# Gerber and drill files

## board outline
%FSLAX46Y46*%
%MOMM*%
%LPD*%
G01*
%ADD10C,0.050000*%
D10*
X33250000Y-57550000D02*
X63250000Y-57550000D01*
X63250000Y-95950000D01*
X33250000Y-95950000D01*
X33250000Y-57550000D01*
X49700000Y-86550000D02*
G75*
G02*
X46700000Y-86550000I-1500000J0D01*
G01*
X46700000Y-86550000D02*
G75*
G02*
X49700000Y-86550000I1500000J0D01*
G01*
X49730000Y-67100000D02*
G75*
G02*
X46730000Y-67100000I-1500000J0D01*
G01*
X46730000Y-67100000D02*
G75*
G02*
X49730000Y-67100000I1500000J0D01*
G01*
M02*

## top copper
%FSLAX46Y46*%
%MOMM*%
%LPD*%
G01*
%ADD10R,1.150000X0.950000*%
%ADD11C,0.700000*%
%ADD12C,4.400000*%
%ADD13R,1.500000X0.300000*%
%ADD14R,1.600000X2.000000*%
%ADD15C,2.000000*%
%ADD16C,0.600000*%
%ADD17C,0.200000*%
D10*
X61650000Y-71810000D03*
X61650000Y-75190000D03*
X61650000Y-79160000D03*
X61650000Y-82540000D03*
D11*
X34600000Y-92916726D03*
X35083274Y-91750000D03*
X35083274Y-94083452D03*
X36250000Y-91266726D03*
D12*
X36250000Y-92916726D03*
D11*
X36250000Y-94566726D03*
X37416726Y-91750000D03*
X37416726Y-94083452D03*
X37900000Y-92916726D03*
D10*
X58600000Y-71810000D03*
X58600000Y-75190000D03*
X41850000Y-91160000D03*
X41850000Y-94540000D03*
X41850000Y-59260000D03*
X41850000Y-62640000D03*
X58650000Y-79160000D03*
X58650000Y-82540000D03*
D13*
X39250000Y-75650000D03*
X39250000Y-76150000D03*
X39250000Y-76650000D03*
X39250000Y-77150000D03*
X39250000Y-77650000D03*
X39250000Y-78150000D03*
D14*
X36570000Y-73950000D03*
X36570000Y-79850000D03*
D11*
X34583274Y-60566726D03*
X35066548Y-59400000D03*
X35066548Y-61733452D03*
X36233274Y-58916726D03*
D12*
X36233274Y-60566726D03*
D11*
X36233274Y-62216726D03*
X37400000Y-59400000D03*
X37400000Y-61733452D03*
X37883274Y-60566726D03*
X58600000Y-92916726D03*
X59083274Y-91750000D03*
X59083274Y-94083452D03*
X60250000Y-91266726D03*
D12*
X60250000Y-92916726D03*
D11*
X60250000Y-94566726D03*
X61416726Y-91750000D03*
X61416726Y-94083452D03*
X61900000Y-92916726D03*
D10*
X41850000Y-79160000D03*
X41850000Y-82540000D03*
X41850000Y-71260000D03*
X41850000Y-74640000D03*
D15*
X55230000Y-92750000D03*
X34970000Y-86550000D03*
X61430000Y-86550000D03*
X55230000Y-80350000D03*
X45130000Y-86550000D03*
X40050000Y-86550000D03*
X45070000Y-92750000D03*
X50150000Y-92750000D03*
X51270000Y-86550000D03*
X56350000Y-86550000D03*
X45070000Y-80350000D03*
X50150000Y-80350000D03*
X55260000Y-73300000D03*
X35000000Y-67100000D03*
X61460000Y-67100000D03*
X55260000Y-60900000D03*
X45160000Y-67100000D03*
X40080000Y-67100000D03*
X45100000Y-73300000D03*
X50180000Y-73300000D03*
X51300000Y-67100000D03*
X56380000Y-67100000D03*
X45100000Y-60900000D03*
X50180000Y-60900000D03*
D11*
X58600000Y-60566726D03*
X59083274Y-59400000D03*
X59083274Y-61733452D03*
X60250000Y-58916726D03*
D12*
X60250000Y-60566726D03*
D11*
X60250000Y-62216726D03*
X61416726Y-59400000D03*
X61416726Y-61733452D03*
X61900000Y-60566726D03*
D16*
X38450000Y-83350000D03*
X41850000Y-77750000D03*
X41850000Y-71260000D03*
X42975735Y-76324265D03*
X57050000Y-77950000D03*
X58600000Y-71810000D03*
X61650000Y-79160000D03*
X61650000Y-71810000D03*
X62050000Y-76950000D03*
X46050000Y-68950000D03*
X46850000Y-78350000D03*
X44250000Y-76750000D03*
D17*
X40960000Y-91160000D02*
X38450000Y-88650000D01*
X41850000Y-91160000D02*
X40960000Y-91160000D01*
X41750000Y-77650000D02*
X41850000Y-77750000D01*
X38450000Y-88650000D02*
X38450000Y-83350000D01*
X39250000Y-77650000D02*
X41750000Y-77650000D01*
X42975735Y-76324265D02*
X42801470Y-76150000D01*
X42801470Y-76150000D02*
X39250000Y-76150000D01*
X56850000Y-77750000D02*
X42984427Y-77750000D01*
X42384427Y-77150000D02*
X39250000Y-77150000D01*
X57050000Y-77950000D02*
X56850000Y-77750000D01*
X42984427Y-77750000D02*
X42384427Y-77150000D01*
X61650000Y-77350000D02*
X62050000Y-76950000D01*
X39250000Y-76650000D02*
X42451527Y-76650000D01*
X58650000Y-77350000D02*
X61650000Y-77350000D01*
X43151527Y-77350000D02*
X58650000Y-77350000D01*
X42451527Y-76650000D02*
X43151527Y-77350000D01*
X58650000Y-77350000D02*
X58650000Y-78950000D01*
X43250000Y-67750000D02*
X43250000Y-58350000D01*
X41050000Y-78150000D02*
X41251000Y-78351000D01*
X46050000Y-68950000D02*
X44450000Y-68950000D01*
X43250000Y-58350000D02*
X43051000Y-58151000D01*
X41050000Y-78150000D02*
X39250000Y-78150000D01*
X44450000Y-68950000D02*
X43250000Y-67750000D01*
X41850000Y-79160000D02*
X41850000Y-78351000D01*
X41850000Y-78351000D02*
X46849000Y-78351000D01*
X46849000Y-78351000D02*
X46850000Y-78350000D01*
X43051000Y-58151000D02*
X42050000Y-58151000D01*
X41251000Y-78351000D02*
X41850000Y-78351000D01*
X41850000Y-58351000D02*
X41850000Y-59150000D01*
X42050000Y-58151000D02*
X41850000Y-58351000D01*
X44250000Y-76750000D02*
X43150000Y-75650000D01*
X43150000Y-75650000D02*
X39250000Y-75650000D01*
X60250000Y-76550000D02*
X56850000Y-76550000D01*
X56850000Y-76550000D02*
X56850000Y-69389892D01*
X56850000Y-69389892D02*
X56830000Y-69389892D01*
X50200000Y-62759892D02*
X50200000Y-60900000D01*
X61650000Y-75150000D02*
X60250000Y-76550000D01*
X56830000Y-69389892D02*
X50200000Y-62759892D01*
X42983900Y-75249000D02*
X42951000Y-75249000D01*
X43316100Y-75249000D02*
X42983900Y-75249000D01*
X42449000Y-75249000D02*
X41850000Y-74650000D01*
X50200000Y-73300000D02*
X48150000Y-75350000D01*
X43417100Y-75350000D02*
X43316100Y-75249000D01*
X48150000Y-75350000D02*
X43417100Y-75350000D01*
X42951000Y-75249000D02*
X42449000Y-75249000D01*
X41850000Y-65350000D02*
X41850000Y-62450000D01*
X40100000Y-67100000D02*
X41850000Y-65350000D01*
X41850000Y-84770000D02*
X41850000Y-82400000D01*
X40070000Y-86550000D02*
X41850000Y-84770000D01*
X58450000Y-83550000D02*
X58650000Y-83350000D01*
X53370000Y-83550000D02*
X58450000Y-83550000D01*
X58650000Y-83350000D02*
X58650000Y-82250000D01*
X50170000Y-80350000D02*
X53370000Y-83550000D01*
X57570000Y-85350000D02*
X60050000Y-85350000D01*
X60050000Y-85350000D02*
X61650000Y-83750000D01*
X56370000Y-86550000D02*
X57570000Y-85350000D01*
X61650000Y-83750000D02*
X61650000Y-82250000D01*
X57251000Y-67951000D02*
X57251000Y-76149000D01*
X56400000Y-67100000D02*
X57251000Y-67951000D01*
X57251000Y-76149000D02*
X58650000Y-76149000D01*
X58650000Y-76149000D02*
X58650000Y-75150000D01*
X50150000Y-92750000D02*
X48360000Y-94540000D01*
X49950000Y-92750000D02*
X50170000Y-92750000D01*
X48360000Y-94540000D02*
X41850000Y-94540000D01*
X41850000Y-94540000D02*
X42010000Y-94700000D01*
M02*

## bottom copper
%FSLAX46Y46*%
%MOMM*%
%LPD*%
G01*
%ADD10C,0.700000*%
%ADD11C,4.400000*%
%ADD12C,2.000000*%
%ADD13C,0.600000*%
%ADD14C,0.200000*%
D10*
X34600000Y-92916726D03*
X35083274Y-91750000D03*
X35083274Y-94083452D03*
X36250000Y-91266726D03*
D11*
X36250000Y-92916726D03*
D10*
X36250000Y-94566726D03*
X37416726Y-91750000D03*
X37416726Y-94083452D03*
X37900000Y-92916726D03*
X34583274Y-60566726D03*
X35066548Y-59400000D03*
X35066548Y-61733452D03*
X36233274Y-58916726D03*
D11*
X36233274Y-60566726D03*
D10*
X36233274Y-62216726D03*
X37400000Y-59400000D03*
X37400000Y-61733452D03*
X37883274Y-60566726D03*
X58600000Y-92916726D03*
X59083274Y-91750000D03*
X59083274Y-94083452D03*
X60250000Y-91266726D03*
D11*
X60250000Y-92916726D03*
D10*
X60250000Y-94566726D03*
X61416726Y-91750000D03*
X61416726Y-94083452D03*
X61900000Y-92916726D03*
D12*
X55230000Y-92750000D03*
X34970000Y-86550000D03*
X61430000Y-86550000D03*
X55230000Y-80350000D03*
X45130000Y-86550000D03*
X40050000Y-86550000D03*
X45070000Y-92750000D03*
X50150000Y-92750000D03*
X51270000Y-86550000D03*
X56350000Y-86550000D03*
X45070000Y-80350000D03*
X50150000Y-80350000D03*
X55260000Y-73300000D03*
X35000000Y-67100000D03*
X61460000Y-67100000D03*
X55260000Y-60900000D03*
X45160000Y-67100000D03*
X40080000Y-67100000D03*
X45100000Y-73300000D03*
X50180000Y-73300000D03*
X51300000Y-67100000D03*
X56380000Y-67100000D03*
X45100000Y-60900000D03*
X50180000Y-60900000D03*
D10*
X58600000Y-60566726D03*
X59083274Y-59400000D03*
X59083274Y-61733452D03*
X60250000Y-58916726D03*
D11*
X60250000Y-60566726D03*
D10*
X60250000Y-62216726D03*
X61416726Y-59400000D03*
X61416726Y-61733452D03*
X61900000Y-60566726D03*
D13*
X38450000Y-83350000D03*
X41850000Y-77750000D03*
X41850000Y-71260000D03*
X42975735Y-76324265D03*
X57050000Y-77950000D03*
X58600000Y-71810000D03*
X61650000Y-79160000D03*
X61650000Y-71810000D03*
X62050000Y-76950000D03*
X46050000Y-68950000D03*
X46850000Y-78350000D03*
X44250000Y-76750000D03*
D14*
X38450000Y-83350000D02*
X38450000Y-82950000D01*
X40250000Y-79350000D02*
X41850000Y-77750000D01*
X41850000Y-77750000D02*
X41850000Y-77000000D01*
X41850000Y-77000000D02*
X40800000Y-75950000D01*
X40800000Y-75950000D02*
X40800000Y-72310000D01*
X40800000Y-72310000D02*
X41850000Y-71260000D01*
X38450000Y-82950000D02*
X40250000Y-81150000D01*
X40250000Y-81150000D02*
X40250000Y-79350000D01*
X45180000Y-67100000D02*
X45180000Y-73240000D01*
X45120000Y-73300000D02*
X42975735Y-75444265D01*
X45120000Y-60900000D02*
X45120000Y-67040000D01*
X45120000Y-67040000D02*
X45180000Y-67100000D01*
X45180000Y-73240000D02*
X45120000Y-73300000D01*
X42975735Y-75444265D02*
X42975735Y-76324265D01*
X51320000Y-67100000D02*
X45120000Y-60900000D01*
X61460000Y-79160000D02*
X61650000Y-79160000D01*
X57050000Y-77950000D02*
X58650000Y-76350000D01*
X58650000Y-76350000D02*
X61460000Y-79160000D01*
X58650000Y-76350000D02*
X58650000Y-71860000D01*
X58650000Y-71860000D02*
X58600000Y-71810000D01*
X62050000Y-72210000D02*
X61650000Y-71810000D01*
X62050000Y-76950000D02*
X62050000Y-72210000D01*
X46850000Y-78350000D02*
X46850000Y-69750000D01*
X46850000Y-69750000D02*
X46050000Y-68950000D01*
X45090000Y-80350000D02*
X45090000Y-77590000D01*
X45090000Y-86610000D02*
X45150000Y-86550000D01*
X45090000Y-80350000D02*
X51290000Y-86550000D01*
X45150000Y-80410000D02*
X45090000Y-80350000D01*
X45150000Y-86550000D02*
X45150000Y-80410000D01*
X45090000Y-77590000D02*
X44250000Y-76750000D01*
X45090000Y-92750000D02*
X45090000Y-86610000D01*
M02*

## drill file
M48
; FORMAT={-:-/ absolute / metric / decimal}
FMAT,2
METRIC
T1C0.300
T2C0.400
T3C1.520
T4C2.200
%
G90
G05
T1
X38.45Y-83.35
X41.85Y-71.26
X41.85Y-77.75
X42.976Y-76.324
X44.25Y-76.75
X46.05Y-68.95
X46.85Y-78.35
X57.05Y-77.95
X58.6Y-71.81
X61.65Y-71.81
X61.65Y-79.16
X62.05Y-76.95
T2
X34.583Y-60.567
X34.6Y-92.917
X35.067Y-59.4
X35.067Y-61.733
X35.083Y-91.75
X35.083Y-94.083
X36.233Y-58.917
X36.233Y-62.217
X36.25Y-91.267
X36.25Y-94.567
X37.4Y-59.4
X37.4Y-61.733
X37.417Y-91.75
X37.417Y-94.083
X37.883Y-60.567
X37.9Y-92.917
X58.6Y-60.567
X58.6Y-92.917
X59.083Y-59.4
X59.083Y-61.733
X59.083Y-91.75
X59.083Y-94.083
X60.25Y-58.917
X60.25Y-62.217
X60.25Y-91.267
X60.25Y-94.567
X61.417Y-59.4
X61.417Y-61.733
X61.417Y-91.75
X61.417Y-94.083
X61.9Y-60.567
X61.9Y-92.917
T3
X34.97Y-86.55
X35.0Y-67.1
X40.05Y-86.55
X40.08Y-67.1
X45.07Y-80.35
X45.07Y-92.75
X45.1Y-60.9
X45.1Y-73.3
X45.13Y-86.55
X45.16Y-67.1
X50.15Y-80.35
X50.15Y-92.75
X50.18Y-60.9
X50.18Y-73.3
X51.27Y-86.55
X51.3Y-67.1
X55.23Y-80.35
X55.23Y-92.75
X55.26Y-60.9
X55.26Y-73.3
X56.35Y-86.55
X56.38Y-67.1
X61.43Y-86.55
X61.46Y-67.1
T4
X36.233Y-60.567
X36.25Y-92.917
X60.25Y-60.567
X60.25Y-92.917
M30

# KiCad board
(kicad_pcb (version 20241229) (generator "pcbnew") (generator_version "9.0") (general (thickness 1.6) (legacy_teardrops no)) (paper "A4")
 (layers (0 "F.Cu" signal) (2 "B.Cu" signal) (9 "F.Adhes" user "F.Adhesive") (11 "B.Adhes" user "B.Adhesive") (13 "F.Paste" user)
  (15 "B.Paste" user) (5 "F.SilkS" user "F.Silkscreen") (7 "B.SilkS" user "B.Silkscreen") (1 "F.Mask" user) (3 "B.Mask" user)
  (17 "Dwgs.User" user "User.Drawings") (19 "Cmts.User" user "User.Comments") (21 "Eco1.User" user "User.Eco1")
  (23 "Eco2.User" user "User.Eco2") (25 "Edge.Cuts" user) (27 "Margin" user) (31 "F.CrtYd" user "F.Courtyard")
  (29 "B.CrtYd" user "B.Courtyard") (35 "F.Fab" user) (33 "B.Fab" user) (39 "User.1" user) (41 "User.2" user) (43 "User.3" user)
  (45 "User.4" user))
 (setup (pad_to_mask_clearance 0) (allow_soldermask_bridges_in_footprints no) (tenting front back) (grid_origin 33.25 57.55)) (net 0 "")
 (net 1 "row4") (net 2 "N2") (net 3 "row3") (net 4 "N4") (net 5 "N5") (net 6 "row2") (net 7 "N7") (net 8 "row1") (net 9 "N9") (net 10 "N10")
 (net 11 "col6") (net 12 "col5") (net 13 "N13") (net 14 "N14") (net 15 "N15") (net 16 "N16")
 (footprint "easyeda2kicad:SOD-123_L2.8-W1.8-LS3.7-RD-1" (layer "F.Cu") (at 61.65 73.5 -90)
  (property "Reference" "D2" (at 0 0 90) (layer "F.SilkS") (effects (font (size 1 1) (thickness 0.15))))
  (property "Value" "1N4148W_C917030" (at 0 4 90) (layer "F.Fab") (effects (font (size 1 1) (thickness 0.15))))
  (pad "1" smd rect (at -1.69 0 270) (size 0.95 1.15) (layers "F.Cu" "F.Mask" "F.Paste") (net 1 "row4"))
  (pad "2" smd rect (at 1.69 0 270) (size 0.95 1.15) (layers "F.Cu" "F.Mask" "F.Paste") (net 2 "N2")))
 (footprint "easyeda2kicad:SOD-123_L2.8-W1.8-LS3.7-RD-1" (layer "F.Cu") (at 61.65 80.85 -90)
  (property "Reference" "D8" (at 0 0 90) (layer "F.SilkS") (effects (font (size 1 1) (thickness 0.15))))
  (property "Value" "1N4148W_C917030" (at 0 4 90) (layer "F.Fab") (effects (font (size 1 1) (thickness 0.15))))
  (pad "1" smd rect (at -1.69 0 270) (size 0.95 1.15) (layers "F.Cu" "F.Mask" "F.Paste") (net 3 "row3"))
  (pad "2" smd rect (at 1.69 0 270) (size 0.95 1.15) (layers "F.Cu" "F.Mask" "F.Paste") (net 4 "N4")))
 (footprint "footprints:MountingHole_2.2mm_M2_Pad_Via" (layer "F.Cu") (at 36.25 92.916726)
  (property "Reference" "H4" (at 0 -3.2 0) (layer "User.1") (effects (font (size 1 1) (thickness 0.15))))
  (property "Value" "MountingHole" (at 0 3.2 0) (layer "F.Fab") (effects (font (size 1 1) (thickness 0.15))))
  (pad "1" thru_hole circle (at -1.65 0) (size 0.7 0.7) (drill 0.4) (layers "*.Cu" "*.Mask") (remove_unused_layers no) (zone_connect 2))
  (pad "1" thru_hole circle (at -1.166726 -1.166726) (size 0.7 0.7) (drill 0.4) (layers "*.Cu" "*.Mask") (remove_unused_layers no)
   (zone_connect 2))
  (pad "1" thru_hole circle (at -1.166726 1.166726) (size 0.7 0.7) (drill 0.4) (layers "*.Cu" "*.Mask") (remove_unused_layers no)
   (zone_connect 2))
  (pad "1" thru_hole circle (at 0 -1.65) (size 0.7 0.7) (drill 0.4) (layers "*.Cu" "*.Mask") (remove_unused_layers no) (zone_connect 2))
  (pad "1" thru_hole circle (at 0 0) (size 4.4 4.4) (drill 2.2) (layers "*.Cu" "*.Mask") (remove_unused_layers no))
  (pad "1" thru_hole circle (at 0 1.65) (size 0.7 0.7) (drill 0.4) (layers "*.Cu" "*.Mask") (remove_unused_layers no) (zone_connect 2))
  (pad "1" thru_hole circle (at 1.166726 -1.166726) (size 0.7 0.7) (drill 0.4) (layers "*.Cu" "*.Mask") (remove_unused_layers no)
   (zone_connect 2))
  (pad "1" thru_hole circle (at 1.166726 1.166726) (size 0.7 0.7) (drill 0.4) (layers "*.Cu" "*.Mask") (remove_unused_layers no)
   (zone_connect 2))
  (pad "1" thru_hole circle (at 1.65 0) (size 0.7 0.7) (drill 0.4) (layers "*.Cu" "*.Mask") (remove_unused_layers no) (zone_connect 2)))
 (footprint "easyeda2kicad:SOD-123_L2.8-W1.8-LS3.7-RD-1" (layer "F.Cu") (at 58.6 73.5 -90)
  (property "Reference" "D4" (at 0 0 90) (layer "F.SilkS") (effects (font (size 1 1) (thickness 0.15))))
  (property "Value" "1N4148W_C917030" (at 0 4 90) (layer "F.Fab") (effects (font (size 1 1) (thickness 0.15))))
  (pad "1" smd rect (at -1.69 0 270) (size 0.95 1.15) (layers "F.Cu" "F.Mask" "F.Paste") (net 3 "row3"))
  (pad "2" smd rect (at 1.69 0 270) (size 0.95 1.15) (layers "F.Cu" "F.Mask" "F.Paste") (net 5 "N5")))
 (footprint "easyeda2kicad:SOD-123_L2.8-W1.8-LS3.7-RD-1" (layer "F.Cu") (at 41.85 92.85 -90)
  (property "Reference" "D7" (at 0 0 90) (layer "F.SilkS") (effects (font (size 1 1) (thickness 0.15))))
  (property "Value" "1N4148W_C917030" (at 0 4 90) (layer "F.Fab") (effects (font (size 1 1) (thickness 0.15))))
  (pad "1" smd rect (at -1.69 0 270) (size 0.95 1.15) (layers "F.Cu" "F.Mask" "F.Paste") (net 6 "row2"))
  (pad "2" smd rect (at 1.69 0 270) (size 0.95 1.15) (layers "F.Cu" "F.Mask" "F.Paste") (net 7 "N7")))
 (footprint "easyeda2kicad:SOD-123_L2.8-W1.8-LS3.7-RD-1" (layer "F.Cu") (at 41.85 60.95 -90)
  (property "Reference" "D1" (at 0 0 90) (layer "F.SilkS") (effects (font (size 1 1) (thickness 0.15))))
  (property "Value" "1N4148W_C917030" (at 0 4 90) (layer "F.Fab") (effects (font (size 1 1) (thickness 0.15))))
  (pad "1" smd rect (at -1.69 0 270) (size 0.95 1.15) (layers "F.Cu" "F.Mask" "F.Paste") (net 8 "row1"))
  (pad "2" smd rect (at 1.69 0 270) (size 0.95 1.15) (layers "F.Cu" "F.Mask" "F.Paste") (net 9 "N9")))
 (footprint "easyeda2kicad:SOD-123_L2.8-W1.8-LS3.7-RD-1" (layer "F.Cu") (at 58.65 80.85 -90)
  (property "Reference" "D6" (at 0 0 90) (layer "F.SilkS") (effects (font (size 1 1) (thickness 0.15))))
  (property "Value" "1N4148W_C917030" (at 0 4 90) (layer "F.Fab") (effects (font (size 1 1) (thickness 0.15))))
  (pad "1" smd rect (at -1.69 0 270) (size 0.95 1.15) (layers "F.Cu" "F.Mask" "F.Paste") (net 1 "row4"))
  (pad "2" smd rect (at 1.69 0 270) (size 0.95 1.15) (layers "F.Cu" "F.Mask" "F.Paste") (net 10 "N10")))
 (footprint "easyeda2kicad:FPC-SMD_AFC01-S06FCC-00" (layer "F.Cu") (at 37.91 76.9 -90)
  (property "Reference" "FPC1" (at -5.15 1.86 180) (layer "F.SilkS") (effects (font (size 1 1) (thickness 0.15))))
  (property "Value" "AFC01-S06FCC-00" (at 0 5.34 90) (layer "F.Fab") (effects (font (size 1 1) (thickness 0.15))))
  (pad "1" smd rect (at -1.25 -1.34 270) (size 0.3 1.5) (layers "F.Cu" "F.Mask" "F.Paste") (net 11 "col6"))
  (pad "2" smd rect (at -0.75 -1.34 270) (size 0.3 1.5) (layers "F.Cu" "F.Mask" "F.Paste") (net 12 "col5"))
  (pad "3" smd rect (at -0.25 -1.34 270) (size 0.3 1.5) (layers "F.Cu" "F.Mask" "F.Paste") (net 1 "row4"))
  (pad "4" smd rect (at 0.25 -1.34 270) (size 0.3 1.5) (layers "F.Cu" "F.Mask" "F.Paste") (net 3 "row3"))
  (pad "5" smd rect (at 0.75 -1.34 270) (size 0.3 1.5) (layers "F.Cu" "F.Mask" "F.Paste") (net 6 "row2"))
  (pad "6" smd rect (at 1.25 -1.34 270) (size 0.3 1.5) (layers "F.Cu" "F.Mask" "F.Paste") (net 8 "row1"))
  (pad "7" smd rect (at -2.95 1.34 270) (size 2 1.6) (layers "F.Cu" "F.Mask" "F.Paste") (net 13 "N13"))
  (pad "8" smd rect (at 2.95 1.34 90) (size 2 1.6) (layers "F.Cu" "F.Mask" "F.Paste") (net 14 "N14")))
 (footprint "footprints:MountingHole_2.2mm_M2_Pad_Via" (layer "F.Cu") (at 36.233274 60.566726)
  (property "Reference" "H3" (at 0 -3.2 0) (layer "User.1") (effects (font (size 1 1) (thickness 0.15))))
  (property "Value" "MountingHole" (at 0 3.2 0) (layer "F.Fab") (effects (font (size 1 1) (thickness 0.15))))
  (pad "1" thru_hole circle (at -1.65 0) (size 0.7 0.7) (drill 0.4) (layers "*.Cu" "*.Mask") (remove_unused_layers no) (zone_connect 2))
  (pad "1" thru_hole circle (at -1.166726 -1.166726) (size 0.7 0.7) (drill 0.4) (layers "*.Cu" "*.Mask") (remove_unused_layers no)
   (zone_connect 2))
  (pad "1" thru_hole circle (at -1.166726 1.166726) (size 0.7 0.7) (drill 0.4) (layers "*.Cu" "*.Mask") (remove_unused_layers no)
   (zone_connect 2))
  (pad "1" thru_hole circle (at 0 -1.65) (size 0.7 0.7) (drill 0.4) (layers "*.Cu" "*.Mask") (remove_unused_layers no) (zone_connect 2))
  (pad "1" thru_hole circle (at 0 0) (size 4.4 4.4) (drill 2.2) (layers "*.Cu" "*.Mask") (remove_unused_layers no))
  (pad "1" thru_hole circle (at 0 1.65) (size 0.7 0.7) (drill 0.4) (layers "*.Cu" "*.Mask") (remove_unused_layers no) (zone_connect 2))
  (pad "1" thru_hole circle (at 1.166726 -1.166726) (size 0.7 0.7) (drill 0.4) (layers "*.Cu" "*.Mask") (remove_unused_layers no)
   (zone_connect 2))
  (pad "1" thru_hole circle (at 1.166726 1.166726) (size 0.7 0.7) (drill 0.4) (layers "*.Cu" "*.Mask") (remove_unused_layers no)
   (zone_connect 2))
  (pad "1" thru_hole circle (at 1.65 0) (size 0.7 0.7) (drill 0.4) (layers "*.Cu" "*.Mask") (remove_unused_layers no) (zone_connect 2)))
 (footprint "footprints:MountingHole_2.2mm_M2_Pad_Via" (layer "F.Cu") (at 60.25 92.916726)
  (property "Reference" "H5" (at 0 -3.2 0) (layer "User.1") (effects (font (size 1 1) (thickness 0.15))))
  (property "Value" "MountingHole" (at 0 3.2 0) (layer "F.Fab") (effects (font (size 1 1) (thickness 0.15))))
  (pad "1" thru_hole circle (at -1.65 0) (size 0.7 0.7) (drill 0.4) (layers "*.Cu" "*.Mask") (remove_unused_layers no) (zone_connect 2))
  (pad "1" thru_hole circle (at -1.166726 -1.166726) (size 0.7 0.7) (drill 0.4) (layers "*.Cu" "*.Mask") (remove_unused_layers no)
   (zone_connect 2))
  (pad "1" thru_hole circle (at -1.166726 1.166726) (size 0.7 0.7) (drill 0.4) (layers "*.Cu" "*.Mask") (remove_unused_layers no)
   (zone_connect 2))
  (pad "1" thru_hole circle (at 0 -1.65) (size 0.7 0.7) (drill 0.4) (layers "*.Cu" "*.Mask") (remove_unused_layers no) (zone_connect 2))
  (pad "1" thru_hole circle (at 0 0) (size 4.4 4.4) (drill 2.2) (layers "*.Cu" "*.Mask") (remove_unused_layers no))
  (pad "1" thru_hole circle (at 0 1.65) (size 0.7 0.7) (drill 0.4) (layers "*.Cu" "*.Mask") (remove_unused_layers no) (zone_connect 2))
  (pad "1" thru_hole circle (at 1.166726 -1.166726) (size 0.7 0.7) (drill 0.4) (layers "*.Cu" "*.Mask") (remove_unused_layers no)
   (zone_connect 2))
  (pad "1" thru_hole circle (at 1.166726 1.166726) (size 0.7 0.7) (drill 0.4) (layers "*.Cu" "*.Mask") (remove_unused_layers no)
   (zone_connect 2))
  (pad "1" thru_hole circle (at 1.65 0) (size 0.7 0.7) (drill 0.4) (layers "*.Cu" "*.Mask") (remove_unused_layers no) (zone_connect 2)))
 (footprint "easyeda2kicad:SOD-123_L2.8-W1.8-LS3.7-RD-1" (layer "F.Cu") (at 41.85 80.85 -90)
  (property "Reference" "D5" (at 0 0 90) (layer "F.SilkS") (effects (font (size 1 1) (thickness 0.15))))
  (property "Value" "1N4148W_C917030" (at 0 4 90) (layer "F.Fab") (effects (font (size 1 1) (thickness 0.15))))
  (pad "1" smd rect (at -1.69 0 270) (size 0.95 1.15) (layers "F.Cu" "F.Mask" "F.Paste") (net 8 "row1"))
  (pad "2" smd rect (at 1.69 0 270) (size 0.95 1.15) (layers "F.Cu" "F.Mask" "F.Paste") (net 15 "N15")))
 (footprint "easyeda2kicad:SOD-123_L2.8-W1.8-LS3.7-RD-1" (layer "F.Cu") (at 41.85 72.95 -90)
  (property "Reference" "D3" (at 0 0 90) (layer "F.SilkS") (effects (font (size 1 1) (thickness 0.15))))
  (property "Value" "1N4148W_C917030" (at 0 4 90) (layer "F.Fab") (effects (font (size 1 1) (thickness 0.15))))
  (pad "1" smd rect (at -1.69 0 270) (size 0.95 1.15) (layers "F.Cu" "F.Mask" "F.Paste") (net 6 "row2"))
  (pad "2" smd rect (at 1.69 0 270) (size 0.95 1.15) (layers "F.Cu" "F.Mask" "F.Paste") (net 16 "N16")))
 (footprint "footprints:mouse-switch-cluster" (layer "F.Cu") (at 48.2 86.55 90)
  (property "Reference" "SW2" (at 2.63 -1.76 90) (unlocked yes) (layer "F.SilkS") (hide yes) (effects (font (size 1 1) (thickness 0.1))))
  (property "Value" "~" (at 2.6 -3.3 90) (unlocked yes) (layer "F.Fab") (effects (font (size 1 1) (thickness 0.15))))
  (fp_circle (center 0 0) (end 1.5 0) (stroke (width 0.05) (type default)) (fill no) (layer "Edge.Cuts"))
  (pad "" thru_hole circle (at -6.2 7.03 90) (size 2 2) (drill 1.52) (layers "*.Cu" "*.Mask") (remove_unused_layers no))
  (pad "" thru_hole circle (at 0 -13.23 270) (size 2 2) (drill 1.52) (layers "*.Cu" "*.Mask") (remove_unused_layers no))
  (pad "" thru_hole circle (at 0 13.23 90) (size 2 2) (drill 1.52) (layers "*.Cu" "*.Mask") (remove_unused_layers no))
  (pad "" thru_hole circle (at 6.2 7.03 90) (size 2 2) (drill 1.52) (layers "*.Cu" "*.Mask") (remove_unused_layers no))
  (pad "1" thru_hole circle (at 0 -3.07 270) (size 2 2) (drill 1.52) (layers "*.Cu" "*.Mask") (remove_unused_layers no) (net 11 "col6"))
  (pad "2" thru_hole circle (at 0 -8.15 270) (size 2 2) (drill 1.52) (layers "*.Cu" "*.Mask") (remove_unused_layers no) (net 15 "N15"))
  (pad "3" thru_hole circle (at -6.2 -3.13 90) (size 2 2) (drill 1.52) (layers "*.Cu" "*.Mask") (remove_unused_layers no) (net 11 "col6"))
  (pad "4" thru_hole circle (at -6.2 1.95 90) (size 2 2) (drill 1.52) (layers "*.Cu" "*.Mask") (remove_unused_layers no) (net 7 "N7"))
  (pad "5" thru_hole circle (at 0 3.07 90) (size 2 2) (drill 1.52) (layers "*.Cu" "*.Mask") (remove_unused_layers no) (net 11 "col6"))
  (pad "6" thru_hole circle (at 0 8.15 90) (size 2 2) (drill 1.52) (layers "*.Cu" "*.Mask") (remove_unused_layers no) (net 4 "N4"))
  (pad "7" thru_hole circle (at 6.2 -3.13 90) (size 2 2) (drill 1.52) (layers "*.Cu" "*.Mask") (remove_unused_layers no) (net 11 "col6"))
  (pad "8" thru_hole circle (at 6.2 1.95 90) (size 2 2) (drill 1.52) (layers "*.Cu" "*.Mask") (remove_unused_layers no) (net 10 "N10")))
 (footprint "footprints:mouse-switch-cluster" (layer "F.Cu") (at 48.23 67.1 90)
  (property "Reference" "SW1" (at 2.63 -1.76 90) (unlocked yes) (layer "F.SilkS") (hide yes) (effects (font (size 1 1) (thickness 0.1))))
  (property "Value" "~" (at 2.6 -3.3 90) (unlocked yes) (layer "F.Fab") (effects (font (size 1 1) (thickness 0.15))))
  (fp_circle (center 0 0) (end 1.5 0) (stroke (width 0.05) (type default)) (fill no) (layer "Edge.Cuts"))
  (pad "" thru_hole circle (at -6.2 7.03 90) (size 2 2) (drill 1.52) (layers "*.Cu" "*.Mask") (remove_unused_layers no))
  (pad "" thru_hole circle (at 0 -13.23 270) (size 2 2) (drill 1.52) (layers "*.Cu" "*.Mask") (remove_unused_layers no))
  (pad "" thru_hole circle (at 0 13.23 90) (size 2 2) (drill 1.52) (layers "*.Cu" "*.Mask") (remove_unused_layers no))
  (pad "" thru_hole circle (at 6.2 7.03 90) (size 2 2) (drill 1.52) (layers "*.Cu" "*.Mask") (remove_unused_layers no))
  (pad "1" thru_hole circle (at 0 -3.07 270) (size 2 2) (drill 1.52) (layers "*.Cu" "*.Mask") (remove_unused_layers no) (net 12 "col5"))
  (pad "2" thru_hole circle (at 0 -8.15 270) (size 2 2) (drill 1.52) (layers "*.Cu" "*.Mask") (remove_unused_layers no) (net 9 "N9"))
  (pad "3" thru_hole circle (at -6.2 -3.13 90) (size 2 2) (drill 1.52) (layers "*.Cu" "*.Mask") (remove_unused_layers no) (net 12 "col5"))
  (pad "4" thru_hole circle (at -6.2 1.95 90) (size 2 2) (drill 1.52) (layers "*.Cu" "*.Mask") (remove_unused_layers no) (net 16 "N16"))
  (pad "5" thru_hole circle (at 0 3.07 90) (size 2 2) (drill 1.52) (layers "*.Cu" "*.Mask") (remove_unused_layers no) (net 12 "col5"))
  (pad "6" thru_hole circle (at 0 8.15 90) (size 2 2) (drill 1.52) (layers "*.Cu" "*.Mask") (remove_unused_layers no) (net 5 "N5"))
  (pad "7" thru_hole circle (at 6.2 -3.13 90) (size 2 2) (drill 1.52) (layers "*.Cu" "*.Mask") (remove_unused_layers no) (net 12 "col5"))
  (pad "8" thru_hole circle (at 6.2 1.95 90) (size 2 2) (drill 1.52) (layers "*.Cu" "*.Mask") (remove_unused_layers no) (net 2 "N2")))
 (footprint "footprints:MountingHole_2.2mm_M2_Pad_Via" (layer "F.Cu") (at 60.25 60.566726)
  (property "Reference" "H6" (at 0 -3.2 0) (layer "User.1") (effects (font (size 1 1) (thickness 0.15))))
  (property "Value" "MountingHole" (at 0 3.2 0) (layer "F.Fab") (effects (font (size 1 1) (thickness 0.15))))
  (pad "1" thru_hole circle (at -1.65 0) (size 0.7 0.7) (drill 0.4) (layers "*.Cu" "*.Mask") (remove_unused_layers no) (zone_connect 2))
  (pad "1" thru_hole circle (at -1.166726 -1.166726) (size 0.7 0.7) (drill 0.4) (layers "*.Cu" "*.Mask") (remove_unused_layers no)
   (zone_connect 2))
  (pad "1" thru_hole circle (at -1.166726 1.166726) (size 0.7 0.7) (drill 0.4) (layers "*.Cu" "*.Mask") (remove_unused_layers no)
   (zone_connect 2))
  (pad "1" thru_hole circle (at 0 -1.65) (size 0.7 0.7) (drill 0.4) (layers "*.Cu" "*.Mask") (remove_unused_layers no) (zone_connect 2))
  (pad "1" thru_hole circle (at 0 0) (size 4.4 4.4) (drill 2.2) (layers "*.Cu" "*.Mask") (remove_unused_layers no))
  (pad "1" thru_hole circle (at 0 1.65) (size 0.7 0.7) (drill 0.4) (layers "*.Cu" "*.Mask") (remove_unused_layers no) (zone_connect 2))
  (pad "1" thru_hole circle (at 1.166726 -1.166726) (size 0.7 0.7) (drill 0.4) (layers "*.Cu" "*.Mask") (remove_unused_layers no)
   (zone_connect 2))
  (pad "1" thru_hole circle (at 1.166726 1.166726) (size 0.7 0.7) (drill 0.4) (layers "*.Cu" "*.Mask") (remove_unused_layers no)
   (zone_connect 2))
  (pad "1" thru_hole circle (at 1.65 0) (size 0.7 0.7) (drill 0.4) (layers "*.Cu" "*.Mask") (remove_unused_layers no) (zone_connect 2)))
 (gr_rect (start 33.25 57.55) (end 63.25 95.95) (stroke (width 0.05) (type default)) (fill no) (layer "Edge.Cuts"))
 (segment (start 40.96 91.16) (end 38.45 88.65) (width 0.2) (layer "F.Cu") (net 6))
 (segment (start 41.85 91.16) (end 40.96 91.16) (width 0.2) (layer "F.Cu") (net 6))
 (segment (start 41.75 77.65) (end 41.85 77.75) (width 0.2) (layer "F.Cu") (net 6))
 (segment (start 38.45 88.65) (end 38.45 83.35) (width 0.2) (layer "F.Cu") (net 6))
 (segment (start 39.25 77.65) (end 41.75 77.65) (width 0.2) (layer "F.Cu") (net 6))
 (via (at 38.45 83.35) (size 0.6) (drill 0.3) (layers "F.Cu" "B.Cu") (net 6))
 (via (at 41.85 77.75) (size 0.6) (drill 0.3) (layers "F.Cu" "B.Cu") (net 6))
 (via (at 41.85 71.26) (size 0.6) (drill 0.3) (layers "F.Cu" "B.Cu") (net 6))
 (segment (start 38.45 83.35) (end 38.45 82.95) (width 0.2) (layer "B.Cu") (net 6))
 (segment (start 40.25 79.35) (end 41.85 77.75) (width 0.2) (layer "B.Cu") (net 6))
 (segment (start 41.85 77.75) (end 41.85 77) (width 0.2) (layer "B.Cu") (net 6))
 (segment (start 41.85 77) (end 40.8 75.95) (width 0.2) (layer "B.Cu") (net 6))
 (segment (start 40.8 75.95) (end 40.8 72.31) (width 0.2) (layer "B.Cu") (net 6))
 (segment (start 40.8 72.31) (end 41.85 71.26) (width 0.2) (layer "B.Cu") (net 6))
 (segment (start 38.45 82.95) (end 40.25 81.15) (width 0.2) (layer "B.Cu") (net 6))
 (segment (start 40.25 81.15) (end 40.25 79.35) (width 0.2) (layer "B.Cu") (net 6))
 (segment (start 42.975735 76.324265) (end 42.80147 76.15) (width 0.2) (layer "F.Cu") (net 12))
 (segment (start 42.80147 76.15) (end 39.25 76.15) (width 0.2) (layer "F.Cu") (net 12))
 (via (at 42.975735 76.324265) (size 0.6) (drill 0.3) (layers "F.Cu" "B.Cu") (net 12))
 (segment (start 45.18 67.1) (end 45.18 73.24) (width 0.2) (layer "B.Cu") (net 12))
 (segment (start 45.12 73.3) (end 42.975735 75.444265) (width 0.2) (layer "B.Cu") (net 12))
 (segment (start 45.12 60.9) (end 45.12 67.04) (width 0.2) (layer "B.Cu") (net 12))
 (segment (start 45.12 67.04) (end 45.18 67.1) (width 0.2) (layer "B.Cu") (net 12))
 (segment (start 45.18 73.24) (end 45.12 73.3) (width 0.2) (layer "B.Cu") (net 12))
 (segment (start 42.975735 75.444265) (end 42.975735 76.324265) (width 0.2) (layer "B.Cu") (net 12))
 (segment (start 51.32 67.1) (end 45.12 60.9) (width 0.2) (layer "B.Cu") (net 12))
 (segment (start 56.85 77.75) (end 42.984427 77.75) (width 0.2) (layer "F.Cu") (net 3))
 (segment (start 42.384427 77.15) (end 39.25 77.15) (width 0.2) (layer "F.Cu") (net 3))
 (segment (start 57.05 77.95) (end 56.85 77.75) (width 0.2) (layer "F.Cu") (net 3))
 (segment (start 42.984427 77.75) (end 42.384427 77.15) (width 0.2) (layer "F.Cu") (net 3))
 (via (at 57.05 77.95) (size 0.6) (drill 0.3) (layers "F.Cu" "B.Cu") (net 3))
 (via (at 58.6 71.81) (size 0.6) (drill 0.3) (layers "F.Cu" "B.Cu") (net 3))
 (via (at 61.65 79.16) (size 0.6) (drill 0.3) (layers "F.Cu" "B.Cu") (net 3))
 (segment (start 61.46 79.16) (end 61.65 79.16) (width 0.2) (layer "B.Cu") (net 3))
 (segment (start 57.05 77.95) (end 58.65 76.35) (width 0.2) (layer "B.Cu") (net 3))
 (segment (start 58.65 76.35) (end 61.46 79.16) (width 0.2) (layer "B.Cu") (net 3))
 (segment (start 58.65 76.35) (end 58.65 71.86) (width 0.2) (layer "B.Cu") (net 3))
 (segment (start 58.65 71.86) (end 58.6 71.81) (width 0.2) (layer "B.Cu") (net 3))
 (segment (start 61.65 77.35) (end 62.05 76.95) (width 0.2) (layer "F.Cu") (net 1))
 (segment (start 39.25 76.65) (end 42.451527 76.65) (width 0.2) (layer "F.Cu") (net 1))
 (segment (start 58.65 77.35) (end 61.65 77.35) (width 0.2) (layer "F.Cu") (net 1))
 (segment (start 43.151527 77.35) (end 58.65 77.35) (width 0.2) (layer "F.Cu") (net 1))
 (segment (start 42.451527 76.65) (end 43.151527 77.35) (width 0.2) (layer "F.Cu") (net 1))
 (segment (start 58.65 77.35) (end 58.65 78.95) (width 0.2) (layer "F.Cu") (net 1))
 (via (at 61.65 71.81) (size 0.6) (drill 0.3) (layers "F.Cu" "B.Cu") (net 1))
 (via (at 62.05 76.95) (size 0.6) (drill 0.3) (layers "F.Cu" "B.Cu") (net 1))
 (segment (start 62.05 72.21) (end 61.65 71.81) (width 0.2) (layer "B.Cu") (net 1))
 (segment (start 62.05 76.95) (end 62.05 72.21) (width 0.2) (layer "B.Cu") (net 1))
 (segment (start 43.25 67.75) (end 43.25 58.35) (width 0.2) (layer "F.Cu") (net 8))
 (segment (start 41.05 78.15) (end 41.251 78.351) (width 0.2) (layer "F.Cu") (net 8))
 (segment (start 46.05 68.95) (end 44.45 68.95) (width 0.2) (layer "F.Cu") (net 8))
 (segment (start 43.25 58.35) (end 43.051 58.151) (width 0.2) (layer "F.Cu") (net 8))
 (segment (start 41.05 78.15) (end 39.25 78.15) (width 0.2) (layer "F.Cu") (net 8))
 (segment (start 44.45 68.95) (end 43.25 67.75) (width 0.2) (layer "F.Cu") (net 8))
 (segment (start 41.85 79.16) (end 41.85 78.351) (width 0.2) (layer "F.Cu") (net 8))
 (segment (start 41.85 78.351) (end 46.849 78.351) (width 0.2) (layer "F.Cu") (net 8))
 (segment (start 46.849 78.351) (end 46.85 78.35) (width 0.2) (layer "F.Cu") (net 8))
 (segment (start 43.051 58.151) (end 42.05 58.151) (width 0.2) (layer "F.Cu") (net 8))
 (segment (start 41.251 78.351) (end 41.85 78.351) (width 0.2) (layer "F.Cu") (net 8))
 (segment (start 41.85 58.351) (end 41.85 59.15) (width 0.2) (layer "F.Cu") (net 8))
 (segment (start 42.05 58.151) (end 41.85 58.351) (width 0.2) (layer "F.Cu") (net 8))
 (via (at 46.05 68.95) (size 0.6) (drill 0.3) (layers "F.Cu" "B.Cu") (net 8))
 (via (at 46.85 78.35) (size 0.6) (drill 0.3) (layers "F.Cu" "B.Cu") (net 8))
 (segment (start 46.85 78.35) (end 46.85 69.75) (width 0.2) (layer "B.Cu") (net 8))
 (segment (start 46.85 69.75) (end 46.05 68.95) (width 0.2) (layer "B.Cu") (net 8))
 (segment (start 44.25 76.75) (end 43.15 75.65) (width 0.2) (layer "F.Cu") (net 11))
 (segment (start 43.15 75.65) (end 39.25 75.65) (width 0.2) (layer "F.Cu") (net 11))
 (via (at 44.25 76.75) (size 0.6) (drill 0.3) (layers "F.Cu" "B.Cu") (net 11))
 (segment (start 45.09 80.35) (end 45.09 77.59) (width 0.2) (layer "B.Cu") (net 11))
 (segment (start 45.09 86.61) (end 45.15 86.55) (width 0.2) (layer "B.Cu") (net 11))
 (segment (start 45.09 80.35) (end 51.29 86.55) (width 0.2) (layer "B.Cu") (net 11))
 (segment (start 45.15 80.41) (end 45.09 80.35) (width 0.2) (layer "B.Cu") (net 11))
 (segment (start 45.15 86.55) (end 45.15 80.41) (width 0.2) (layer "B.Cu") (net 11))
 (segment (start 45.09 77.59) (end 44.25 76.75) (width 0.2) (layer "B.Cu") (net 11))
 (segment (start 45.09 92.75) (end 45.09 86.61) (width 0.2) (layer "B.Cu") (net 11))
 (segment (start 60.25 76.55) (end 56.85 76.55) (width 0.2) (layer "F.Cu") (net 2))
 (segment (start 56.85 76.55) (end 56.85 69.389892) (width 0.2) (layer "F.Cu") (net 2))
 (segment (start 56.85 69.389892) (end 56.83 69.389892) (width 0.2) (layer "F.Cu") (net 2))
 (segment (start 50.2 62.759892) (end 50.2 60.9) (width 0.2) (layer "F.Cu") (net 2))
 (segment (start 61.65 75.15) (end 60.25 76.55) (width 0.2) (layer "F.Cu") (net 2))
 (segment (start 56.83 69.389892) (end 50.2 62.759892) (width 0.2) (layer "F.Cu") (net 2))
 (segment (start 42.9839 75.249) (end 42.951 75.249) (width 0.2) (layer "F.Cu") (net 16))
 (segment (start 43.3161 75.249) (end 42.9839 75.249) (width 0.2) (layer "F.Cu") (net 16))
 (segment (start 42.449 75.249) (end 41.85 74.65) (width 0.2) (layer "F.Cu") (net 16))
 (segment (start 50.2 73.3) (end 48.15 75.35) (width 0.2) (layer "F.Cu") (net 16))
 (segment (start 43.4171 75.35) (end 43.3161 75.249) (width 0.2) (layer "F.Cu") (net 16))
 (segment (start 48.15 75.35) (end 43.4171 75.35) (width 0.2) (layer "F.Cu") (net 16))
 (segment (start 42.951 75.249) (end 42.449 75.249) (width 0.2) (layer "F.Cu") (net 16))
 (segment (start 41.85 65.35) (end 41.85 62.45) (width 0.2) (layer "F.Cu") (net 9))
 (segment (start 40.1 67.1) (end 41.85 65.35) (width 0.2) (layer "F.Cu") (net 9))
 (segment (start 41.85 84.77) (end 41.85 82.4) (width 0.2) (layer "F.Cu") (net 15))
 (segment (start 40.07 86.55) (end 41.85 84.77) (width 0.2) (layer "F.Cu") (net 15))
 (segment (start 58.45 83.55) (end 58.65 83.35) (width 0.2) (layer "F.Cu") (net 10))
 (segment (start 53.37 83.55) (end 58.45 83.55) (width 0.2) (layer "F.Cu") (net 10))
 (segment (start 58.65 83.35) (end 58.65 82.25) (width 0.2) (layer "F.Cu") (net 10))
 (segment (start 50.17 80.35) (end 53.37 83.55) (width 0.2) (layer "F.Cu") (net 10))
 (segment (start 57.57 85.35) (end 60.05 85.35) (width 0.2) (layer "F.Cu") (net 4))
 (segment (start 60.05 85.35) (end 61.65 83.75) (width 0.2) (layer "F.Cu") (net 4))
 (segment (start 56.37 86.55) (end 57.57 85.35) (width 0.2) (layer "F.Cu") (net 4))
 (segment (start 61.65 83.75) (end 61.65 82.25) (width 0.2) (layer "F.Cu") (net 4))
 (segment (start 57.251 67.951) (end 57.251 76.149) (width 0.2) (layer "F.Cu") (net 5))
 (segment (start 56.4 67.1) (end 57.251 67.951) (width 0.2) (layer "F.Cu") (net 5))
 (segment (start 57.251 76.149) (end 58.65 76.149) (width 0.2) (layer "F.Cu") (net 5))
 (segment (start 58.65 76.149) (end 58.65 75.15) (width 0.2) (layer "F.Cu") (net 5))
 (segment (start 50.15 92.75) (end 48.36 94.54) (width 0.2) (layer "F.Cu") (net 7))
 (segment (start 49.95 92.75) (end 50.17 92.75) (width 0.2) (layer "F.Cu") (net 7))
 (segment (start 48.36 94.54) (end 41.85 94.54) (width 0.2) (layer "F.Cu") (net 7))
 (segment (start 41.85 94.54) (end 42.01 94.7) (width 0.2) (layer "F.Cu") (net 7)))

